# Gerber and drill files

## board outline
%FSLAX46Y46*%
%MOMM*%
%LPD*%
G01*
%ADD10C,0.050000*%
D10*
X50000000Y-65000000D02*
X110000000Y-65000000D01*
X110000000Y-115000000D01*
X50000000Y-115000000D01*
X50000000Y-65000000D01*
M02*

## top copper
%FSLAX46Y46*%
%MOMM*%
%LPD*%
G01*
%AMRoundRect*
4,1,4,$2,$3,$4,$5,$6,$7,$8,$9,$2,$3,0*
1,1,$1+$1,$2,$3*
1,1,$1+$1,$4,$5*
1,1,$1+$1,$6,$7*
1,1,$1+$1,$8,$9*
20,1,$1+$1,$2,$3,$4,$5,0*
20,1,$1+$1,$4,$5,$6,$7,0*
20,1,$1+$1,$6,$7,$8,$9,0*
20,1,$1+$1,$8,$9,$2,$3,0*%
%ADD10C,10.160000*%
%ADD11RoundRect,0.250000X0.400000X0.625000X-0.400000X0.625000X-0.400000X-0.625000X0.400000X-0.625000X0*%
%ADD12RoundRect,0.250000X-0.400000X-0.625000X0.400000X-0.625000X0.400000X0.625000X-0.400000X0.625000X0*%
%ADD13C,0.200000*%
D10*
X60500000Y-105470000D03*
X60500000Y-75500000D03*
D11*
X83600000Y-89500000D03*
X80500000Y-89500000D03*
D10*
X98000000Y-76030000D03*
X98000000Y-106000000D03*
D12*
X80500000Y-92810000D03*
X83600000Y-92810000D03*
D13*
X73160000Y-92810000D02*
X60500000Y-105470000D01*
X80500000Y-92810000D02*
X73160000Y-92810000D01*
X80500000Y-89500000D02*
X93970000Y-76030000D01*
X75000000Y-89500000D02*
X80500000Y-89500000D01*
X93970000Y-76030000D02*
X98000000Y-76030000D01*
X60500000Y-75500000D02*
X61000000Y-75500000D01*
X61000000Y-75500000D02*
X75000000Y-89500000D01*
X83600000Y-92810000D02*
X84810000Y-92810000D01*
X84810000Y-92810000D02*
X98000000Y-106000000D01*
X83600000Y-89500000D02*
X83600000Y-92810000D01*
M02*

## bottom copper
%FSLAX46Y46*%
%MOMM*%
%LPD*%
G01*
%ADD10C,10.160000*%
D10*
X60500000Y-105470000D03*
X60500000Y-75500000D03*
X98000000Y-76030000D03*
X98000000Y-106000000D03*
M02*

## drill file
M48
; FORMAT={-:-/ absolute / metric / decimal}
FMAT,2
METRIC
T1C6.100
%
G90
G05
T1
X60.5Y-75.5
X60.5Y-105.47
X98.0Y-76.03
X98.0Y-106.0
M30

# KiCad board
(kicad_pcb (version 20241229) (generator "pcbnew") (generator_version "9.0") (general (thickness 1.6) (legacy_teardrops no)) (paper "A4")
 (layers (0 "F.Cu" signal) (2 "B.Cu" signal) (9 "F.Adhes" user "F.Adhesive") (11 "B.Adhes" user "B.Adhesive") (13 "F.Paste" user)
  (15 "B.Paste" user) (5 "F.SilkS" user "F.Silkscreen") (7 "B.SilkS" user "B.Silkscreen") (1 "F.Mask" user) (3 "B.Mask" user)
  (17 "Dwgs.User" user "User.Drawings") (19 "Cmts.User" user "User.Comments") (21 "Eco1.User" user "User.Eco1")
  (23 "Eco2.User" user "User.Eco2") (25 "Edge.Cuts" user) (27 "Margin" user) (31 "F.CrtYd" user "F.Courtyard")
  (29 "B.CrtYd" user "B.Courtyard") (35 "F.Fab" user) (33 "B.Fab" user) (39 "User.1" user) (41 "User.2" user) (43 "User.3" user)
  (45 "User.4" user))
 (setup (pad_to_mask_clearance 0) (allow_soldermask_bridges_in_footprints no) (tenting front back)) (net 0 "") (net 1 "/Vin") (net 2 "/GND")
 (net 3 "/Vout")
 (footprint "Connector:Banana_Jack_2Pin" (layer "F.Cu") (at 60.5 105.47 90)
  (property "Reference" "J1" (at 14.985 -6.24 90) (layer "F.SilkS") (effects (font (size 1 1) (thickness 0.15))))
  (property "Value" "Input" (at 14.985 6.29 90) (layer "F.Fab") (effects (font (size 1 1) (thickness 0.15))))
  (pad "1" thru_hole circle (at 0 0 90) (size 10.16 10.16) (drill 6.1) (layers "*.Cu" "*.Mask") (remove_unused_layers no) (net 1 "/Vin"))
  (pad "2" thru_hole circle (at 29.97 0 90) (size 10.16 10.16) (drill 6.1) (layers "*.Cu" "*.Mask") (remove_unused_layers no) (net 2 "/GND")))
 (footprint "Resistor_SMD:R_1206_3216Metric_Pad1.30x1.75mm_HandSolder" (layer "F.Cu") (at 82.05 89.5 180)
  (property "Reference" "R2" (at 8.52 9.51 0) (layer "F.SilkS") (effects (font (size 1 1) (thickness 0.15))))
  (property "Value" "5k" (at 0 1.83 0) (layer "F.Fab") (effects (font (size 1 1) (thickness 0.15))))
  (pad "1" smd roundrect (at -1.55 0 180) (size 1.3 1.75) (layers "F.Cu" "F.Mask" "F.Paste") (roundrect_rratio 0.192308) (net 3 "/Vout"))
  (pad "2" smd roundrect (at 1.55 0 180) (size 1.3 1.75) (layers "F.Cu" "F.Mask" "F.Paste") (roundrect_rratio 0.192308) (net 2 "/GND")))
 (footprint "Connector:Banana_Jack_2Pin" (layer "F.Cu") (at 98 76.03 -90)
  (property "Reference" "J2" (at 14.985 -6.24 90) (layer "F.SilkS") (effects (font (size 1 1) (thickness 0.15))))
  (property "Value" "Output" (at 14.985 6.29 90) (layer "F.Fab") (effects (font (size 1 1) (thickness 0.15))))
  (pad "1" thru_hole circle (at 0 0 270) (size 10.16 10.16) (drill 6.1) (layers "*.Cu" "*.Mask") (remove_unused_layers no) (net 2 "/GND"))
  (pad "2" thru_hole circle (at 29.97 0 270) (size 10.16 10.16) (drill 6.1) (layers "*.Cu" "*.Mask") (remove_unused_layers no)
   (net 3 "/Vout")))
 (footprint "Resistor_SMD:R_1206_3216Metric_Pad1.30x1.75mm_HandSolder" (layer "F.Cu") (at 82.05 92.81)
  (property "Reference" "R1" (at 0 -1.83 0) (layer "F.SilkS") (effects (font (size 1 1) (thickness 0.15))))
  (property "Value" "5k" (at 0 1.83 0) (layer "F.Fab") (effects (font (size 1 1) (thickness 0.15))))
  (pad "1" smd roundrect (at -1.55 0) (size 1.3 1.75) (layers "F.Cu" "F.Mask" "F.Paste") (roundrect_rratio 0.192308) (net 1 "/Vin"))
  (pad "2" smd roundrect (at 1.55 0) (size 1.3 1.75) (layers "F.Cu" "F.Mask" "F.Paste") (roundrect_rratio 0.192308) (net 3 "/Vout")))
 (gr_rect (start 50 65) (end 110 115) (stroke (width 0.05) (type default)) (fill no) (layer "Edge.Cuts"))
 (segment (start 73.16 92.81) (end 60.5 105.47) (width 0.2) (layer "F.Cu") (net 1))
 (segment (start 80.5 92.81) (end 73.16 92.81) (width 0.2) (layer "F.Cu") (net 1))
 (segment (start 80.5 89.5) (end 93.97 76.03) (width 0.2) (layer "F.Cu") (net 2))
 (segment (start 75 89.5) (end 80.5 89.5) (width 0.2) (layer "F.Cu") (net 2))
 (segment (start 93.97 76.03) (end 98 76.03) (width 0.2) (layer "F.Cu") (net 2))
 (segment (start 60.5 75.5) (end 61 75.5) (width 0.2) (layer "F.Cu") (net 2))
 (segment (start 61 75.5) (end 75 89.5) (width 0.2) (layer "F.Cu") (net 2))
 (segment (start 83.6 92.81) (end 84.81 92.81) (width 0.2) (layer "F.Cu") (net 3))
 (segment (start 84.81 92.81) (end 98 106) (width 0.2) (layer "F.Cu") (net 3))
 (segment (start 83.6 89.5) (end 83.6 92.81) (width 0.2) (layer "F.Cu") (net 3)))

